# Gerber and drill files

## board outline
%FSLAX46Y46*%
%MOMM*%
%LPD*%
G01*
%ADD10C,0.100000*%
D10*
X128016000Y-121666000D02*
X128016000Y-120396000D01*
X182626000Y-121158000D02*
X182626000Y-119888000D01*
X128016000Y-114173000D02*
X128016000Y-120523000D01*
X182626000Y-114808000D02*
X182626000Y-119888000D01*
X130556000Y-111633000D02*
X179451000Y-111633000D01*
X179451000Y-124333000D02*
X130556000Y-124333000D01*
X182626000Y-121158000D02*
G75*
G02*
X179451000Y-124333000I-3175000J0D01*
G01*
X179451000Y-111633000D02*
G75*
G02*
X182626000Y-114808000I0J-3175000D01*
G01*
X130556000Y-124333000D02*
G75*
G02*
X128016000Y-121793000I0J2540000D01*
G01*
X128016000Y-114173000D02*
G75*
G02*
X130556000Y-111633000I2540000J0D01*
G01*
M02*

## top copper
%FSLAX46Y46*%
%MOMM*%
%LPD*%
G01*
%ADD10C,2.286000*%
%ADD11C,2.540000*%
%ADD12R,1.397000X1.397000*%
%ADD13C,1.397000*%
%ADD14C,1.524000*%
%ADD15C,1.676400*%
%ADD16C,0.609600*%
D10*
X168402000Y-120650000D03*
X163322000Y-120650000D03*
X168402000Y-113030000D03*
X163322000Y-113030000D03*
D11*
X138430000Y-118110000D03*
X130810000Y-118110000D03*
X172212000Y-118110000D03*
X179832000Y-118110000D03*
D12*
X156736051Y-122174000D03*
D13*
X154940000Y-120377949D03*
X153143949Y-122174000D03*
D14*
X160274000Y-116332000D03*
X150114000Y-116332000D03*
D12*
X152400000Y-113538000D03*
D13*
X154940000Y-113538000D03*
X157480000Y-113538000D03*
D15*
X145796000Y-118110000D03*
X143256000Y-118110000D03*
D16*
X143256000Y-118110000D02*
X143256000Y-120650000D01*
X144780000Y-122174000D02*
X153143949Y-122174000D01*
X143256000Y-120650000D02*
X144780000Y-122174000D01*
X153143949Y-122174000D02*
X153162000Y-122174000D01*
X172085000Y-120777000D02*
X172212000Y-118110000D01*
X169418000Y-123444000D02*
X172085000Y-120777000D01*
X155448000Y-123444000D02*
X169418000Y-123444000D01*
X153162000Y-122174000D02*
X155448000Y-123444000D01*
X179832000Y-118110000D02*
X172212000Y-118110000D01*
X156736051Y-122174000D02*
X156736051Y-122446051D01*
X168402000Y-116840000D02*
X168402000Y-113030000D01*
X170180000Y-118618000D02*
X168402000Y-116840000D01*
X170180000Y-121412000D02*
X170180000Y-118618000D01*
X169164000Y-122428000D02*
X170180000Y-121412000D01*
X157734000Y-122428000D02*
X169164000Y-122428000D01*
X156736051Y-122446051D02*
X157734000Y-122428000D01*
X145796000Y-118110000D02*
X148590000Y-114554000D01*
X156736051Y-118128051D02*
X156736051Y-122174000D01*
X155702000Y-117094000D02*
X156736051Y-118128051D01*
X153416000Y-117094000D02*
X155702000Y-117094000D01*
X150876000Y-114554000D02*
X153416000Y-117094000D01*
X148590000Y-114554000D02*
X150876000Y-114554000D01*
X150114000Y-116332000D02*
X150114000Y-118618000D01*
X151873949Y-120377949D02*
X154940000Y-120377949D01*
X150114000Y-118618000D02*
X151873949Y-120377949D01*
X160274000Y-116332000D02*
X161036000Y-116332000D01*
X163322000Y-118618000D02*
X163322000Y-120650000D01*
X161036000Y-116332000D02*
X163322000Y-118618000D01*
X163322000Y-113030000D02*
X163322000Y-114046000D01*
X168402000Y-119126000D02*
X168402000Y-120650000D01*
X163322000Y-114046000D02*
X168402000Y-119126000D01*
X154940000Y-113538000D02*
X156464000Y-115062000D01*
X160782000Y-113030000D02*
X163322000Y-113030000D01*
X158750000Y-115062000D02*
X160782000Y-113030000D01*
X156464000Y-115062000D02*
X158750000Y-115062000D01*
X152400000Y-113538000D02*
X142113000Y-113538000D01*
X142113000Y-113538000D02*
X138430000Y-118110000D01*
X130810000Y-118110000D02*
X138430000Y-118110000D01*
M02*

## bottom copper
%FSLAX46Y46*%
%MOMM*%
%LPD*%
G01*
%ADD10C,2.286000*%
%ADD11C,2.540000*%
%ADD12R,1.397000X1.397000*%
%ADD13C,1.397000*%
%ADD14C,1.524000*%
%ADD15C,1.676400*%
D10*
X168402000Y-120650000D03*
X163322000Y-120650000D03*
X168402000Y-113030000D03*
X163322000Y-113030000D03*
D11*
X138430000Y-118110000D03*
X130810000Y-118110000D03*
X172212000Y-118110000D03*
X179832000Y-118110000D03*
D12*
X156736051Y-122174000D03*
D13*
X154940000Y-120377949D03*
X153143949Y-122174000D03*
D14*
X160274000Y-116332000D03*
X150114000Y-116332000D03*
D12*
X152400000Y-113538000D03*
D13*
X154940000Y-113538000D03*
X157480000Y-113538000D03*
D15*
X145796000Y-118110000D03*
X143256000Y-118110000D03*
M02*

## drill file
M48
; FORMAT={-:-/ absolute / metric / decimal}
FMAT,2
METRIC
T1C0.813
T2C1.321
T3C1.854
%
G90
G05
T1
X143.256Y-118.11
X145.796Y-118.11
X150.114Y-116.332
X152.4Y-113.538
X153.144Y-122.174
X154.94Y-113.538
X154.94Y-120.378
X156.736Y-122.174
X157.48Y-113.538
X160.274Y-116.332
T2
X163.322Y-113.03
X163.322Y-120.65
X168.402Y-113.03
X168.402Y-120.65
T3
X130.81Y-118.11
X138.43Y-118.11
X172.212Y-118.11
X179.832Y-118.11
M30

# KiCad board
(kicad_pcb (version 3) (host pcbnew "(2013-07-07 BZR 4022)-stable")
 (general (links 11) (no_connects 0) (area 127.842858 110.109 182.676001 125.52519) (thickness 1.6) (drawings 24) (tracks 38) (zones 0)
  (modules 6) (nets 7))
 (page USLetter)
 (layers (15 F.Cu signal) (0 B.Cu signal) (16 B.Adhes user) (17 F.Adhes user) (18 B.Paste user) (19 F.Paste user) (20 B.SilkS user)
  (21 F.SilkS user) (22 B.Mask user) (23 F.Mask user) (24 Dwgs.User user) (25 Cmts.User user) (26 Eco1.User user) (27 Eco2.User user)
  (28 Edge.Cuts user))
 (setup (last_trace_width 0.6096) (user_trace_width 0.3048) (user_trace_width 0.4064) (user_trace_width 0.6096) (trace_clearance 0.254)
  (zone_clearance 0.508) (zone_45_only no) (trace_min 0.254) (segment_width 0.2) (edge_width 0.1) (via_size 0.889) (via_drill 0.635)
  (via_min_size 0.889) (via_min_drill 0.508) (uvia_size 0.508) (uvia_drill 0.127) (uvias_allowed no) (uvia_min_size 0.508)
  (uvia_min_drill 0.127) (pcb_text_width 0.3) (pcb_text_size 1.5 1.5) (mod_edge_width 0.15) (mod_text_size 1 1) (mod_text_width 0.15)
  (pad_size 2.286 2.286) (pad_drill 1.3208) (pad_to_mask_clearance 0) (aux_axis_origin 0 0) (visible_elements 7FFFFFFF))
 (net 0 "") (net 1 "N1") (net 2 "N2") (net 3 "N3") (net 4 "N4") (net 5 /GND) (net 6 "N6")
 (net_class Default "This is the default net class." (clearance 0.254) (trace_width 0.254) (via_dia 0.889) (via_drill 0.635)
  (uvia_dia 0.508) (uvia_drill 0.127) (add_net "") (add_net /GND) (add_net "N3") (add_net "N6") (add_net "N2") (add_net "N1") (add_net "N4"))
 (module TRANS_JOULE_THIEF (layer F.Cu) (at 165.862 118.11 180)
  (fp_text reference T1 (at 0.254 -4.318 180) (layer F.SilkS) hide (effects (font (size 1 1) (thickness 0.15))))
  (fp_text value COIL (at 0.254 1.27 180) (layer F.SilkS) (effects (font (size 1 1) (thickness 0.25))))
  (pad 1 thru_hole circle (at -2.54 -2.54 180) (size 2.286 2.286) (drill 1.3208) (layers *.Cu *.Mask F.SilkS) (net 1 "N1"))
  (pad 2 thru_hole circle (at 2.54 -2.54 180) (size 2.286 2.286) (drill 1.3208) (layers *.Cu *.Mask F.SilkS) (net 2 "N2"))
  (pad 3 thru_hole circle (at -2.54 5.08 180) (size 2.286 2.286) (drill 1.3208) (layers *.Cu *.Mask F.SilkS) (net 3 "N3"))
  (pad 4 thru_hole circle (at 2.54 5.08 180) (size 2.286 2.286) (drill 1.3208) (layers *.Cu *.Mask F.SilkS) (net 1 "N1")))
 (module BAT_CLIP (layer F.Cu) (at 155.448 118.11)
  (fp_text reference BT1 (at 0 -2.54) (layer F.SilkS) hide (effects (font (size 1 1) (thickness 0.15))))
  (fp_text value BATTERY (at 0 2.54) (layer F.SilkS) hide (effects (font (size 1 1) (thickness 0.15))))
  (pad 1 thru_hole circle (at -17.018 0) (size 2.54 2.54) (drill 1.8542) (layers *.Cu *.Mask F.SilkS) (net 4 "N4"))
  (pad 1 thru_hole circle (at -24.638 0) (size 2.54 2.54) (drill 1.8542) (layers *.Cu *.Mask F.SilkS) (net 4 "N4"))
  (pad 2 thru_hole circle (at 16.764 0) (size 2.54 2.54) (drill 1.8542) (layers *.Cu *.Mask F.SilkS) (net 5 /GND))
  (pad 2 thru_hole circle (at 24.384 0) (size 2.54 2.54) (drill 1.8542) (layers *.Cu *.Mask F.SilkS) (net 5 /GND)))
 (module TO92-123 (layer F.Cu) (at 154.94 122.174 315)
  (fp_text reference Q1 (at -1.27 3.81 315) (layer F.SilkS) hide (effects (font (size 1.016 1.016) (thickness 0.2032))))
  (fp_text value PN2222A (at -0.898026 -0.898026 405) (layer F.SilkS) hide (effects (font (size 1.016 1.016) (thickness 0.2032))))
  (pad 3 thru_hole rect (at 1.27 -1.27) (size 1.397 1.397) (drill 0.8128) (layers *.Cu *.Mask F.SilkS) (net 3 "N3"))
  (pad 2 thru_hole circle (at -1.27 -1.27 315) (size 1.397 1.397) (drill 0.8128) (layers *.Cu *.Mask F.SilkS) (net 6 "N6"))
  (pad 1 thru_hole circle (at -1.27 1.27 315) (size 1.397 1.397) (drill 0.8128) (layers *.Cu *.Mask F.SilkS) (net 5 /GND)))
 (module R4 (layer F.Cu) (at 155.194 116.332 180) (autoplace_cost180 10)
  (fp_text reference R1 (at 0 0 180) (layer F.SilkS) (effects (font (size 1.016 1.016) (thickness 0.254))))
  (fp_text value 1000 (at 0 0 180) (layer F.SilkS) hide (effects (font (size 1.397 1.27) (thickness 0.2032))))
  (pad 1 thru_hole circle (at -5.08 0 180) (size 1.524 1.524) (drill 0.8128) (layers *.Cu *.Mask F.SilkS) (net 2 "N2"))
  (pad 2 thru_hole circle (at 5.08 0 180) (size 1.524 1.524) (drill 0.8128) (layers *.Cu *.Mask F.SilkS) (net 6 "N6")))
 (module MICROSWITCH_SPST (layer F.Cu) (at 154.94 113.538)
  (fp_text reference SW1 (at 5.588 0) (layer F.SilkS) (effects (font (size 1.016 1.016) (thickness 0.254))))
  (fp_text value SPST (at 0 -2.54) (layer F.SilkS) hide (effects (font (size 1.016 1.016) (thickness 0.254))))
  (pad 1 thru_hole rect (at -2.54 0) (size 1.397 1.397) (drill 0.8128) (layers *.Cu *.Mask F.SilkS) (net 4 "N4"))
  (pad 2 thru_hole circle (at 0 0) (size 1.397 1.397) (drill 0.8128) (layers *.Cu *.Mask F.SilkS) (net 1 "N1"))
  (pad 3 thru_hole circle (at 2.54 0) (size 1.397 1.397) (drill 0.8128) (layers *.Cu *.Mask F.SilkS)))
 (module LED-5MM (layer F.Cu) (at 144.526 118.11 180)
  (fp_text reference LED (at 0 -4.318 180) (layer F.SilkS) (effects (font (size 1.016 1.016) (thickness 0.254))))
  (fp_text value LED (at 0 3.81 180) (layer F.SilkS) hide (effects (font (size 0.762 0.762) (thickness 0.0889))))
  (pad 1 thru_hole circle (at -1.27 0 180) (size 1.6764 1.6764) (drill 0.8128) (layers *.Cu *.Mask F.SilkS) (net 3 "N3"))
  (pad 2 thru_hole circle (at 1.27 0 180) (size 1.6764 1.6764) (drill 0.8128) (layers *.Cu *.Mask F.SilkS) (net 5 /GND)))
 (gr_line (start 128.016 121.666) (end 128.016 120.396) (angle 90) (layer Edge.Cuts) (width 0.1))
 (gr_line (start 182.626 121.158) (end 182.626 119.888) (angle 90) (layer Edge.Cuts) (width 0.1))
 (gr_line (start 128.016 114.173) (end 128.016 120.523) (angle 90) (layer Edge.Cuts) (width 0.1))
 (gr_line (start 182.626 114.808) (end 182.626 119.888) (angle 90) (layer Edge.Cuts) (width 0.1))
 (gr_line (start 130.556 111.633) (end 179.451 111.633) (angle 90) (layer Edge.Cuts) (width 0.1))
 (gr_line (start 179.451 124.333) (end 130.556 124.333) (angle 90) (layer Edge.Cuts) (width 0.1))
 (gr_arc (start 179.451 121.158) (end 182.626 121.158) (angle 90) (layer Edge.Cuts) (width 0.1))
 (gr_arc (start 179.451 114.808) (end 179.451 111.633) (angle 90) (layer Edge.Cuts) (width 0.1))
 (gr_arc (start 130.556 121.793) (end 130.556 124.333) (angle 90) (layer Edge.Cuts) (width 0.1))
 (gr_arc (start 130.556 114.173) (end 128.016 114.173) (angle 90) (layer Edge.Cuts) (width 0.1))
 (segment (start 143.256 118.11) (end 143.256 120.65) (width 0.6096) (layer F.Cu) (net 5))
 (segment (start 144.78 122.174) (end 153.143949 122.174) (width 0.6096) (layer F.Cu) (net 5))
 (segment (start 143.256 120.65) (end 144.78 122.174) (width 0.6096) (layer F.Cu) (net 5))
 (segment (start 153.143949 122.174) (end 153.162 122.174) (width 0.6096) (layer F.Cu) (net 5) (status 30))
 (segment (start 172.085 120.777) (end 172.212 118.11) (width 0.6096) (layer F.Cu) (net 5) (status 20))
 (segment (start 169.418 123.444) (end 172.085 120.777) (width 0.6096) (layer F.Cu) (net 5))
 (segment (start 155.448 123.444) (end 169.418 123.444) (width 0.6096) (layer F.Cu) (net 5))
 (segment (start 153.162 122.174) (end 155.448 123.444) (width 0.6096) (layer F.Cu) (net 5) (status 10))
 (segment (start 179.832 118.11) (end 172.212 118.11) (width 0.6096) (layer F.Cu) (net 5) (status 30))
 (segment (start 156.736051 122.174) (end 156.736051 122.446051) (width 0.6096) (layer F.Cu) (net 3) (status 30))
 (segment (start 168.402 116.84) (end 168.402 113.03) (width 0.6096) (layer F.Cu) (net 3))
 (segment (start 170.18 118.618) (end 168.402 116.84) (width 0.6096) (layer F.Cu) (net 3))
 (segment (start 170.18 121.412) (end 170.18 118.618) (width 0.6096) (layer F.Cu) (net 3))
 (segment (start 169.164 122.428) (end 170.18 121.412) (width 0.6096) (layer F.Cu) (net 3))
 (segment (start 157.734 122.428) (end 169.164 122.428) (width 0.6096) (layer F.Cu) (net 3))
 (segment (start 156.736051 122.446051) (end 157.734 122.428) (width 0.6096) (layer F.Cu) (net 3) (status 10))
 (segment (start 145.796 118.11) (end 148.59 114.554) (width 0.6096) (layer F.Cu) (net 3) (status 10))
 (segment (start 156.736051 118.128051) (end 156.736051 122.174) (width 0.6096) (layer F.Cu) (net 3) (status 20))
 (segment (start 155.702 117.094) (end 156.736051 118.128051) (width 0.6096) (layer F.Cu) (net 3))
 (segment (start 153.416 117.094) (end 155.702 117.094) (width 0.6096) (layer F.Cu) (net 3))
 (segment (start 150.876 114.554) (end 153.416 117.094) (width 0.6096) (layer F.Cu) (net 3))
 (segment (start 148.59 114.554) (end 150.876 114.554) (width 0.6096) (layer F.Cu) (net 3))
 (segment (start 150.114 116.332) (end 150.114 118.618) (width 0.6096) (layer F.Cu) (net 6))
 (segment (start 151.873949 120.377949) (end 154.94 120.377949) (width 0.6096) (layer F.Cu) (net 6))
 (segment (start 150.114 118.618) (end 151.873949 120.377949) (width 0.6096) (layer F.Cu) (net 6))
 (segment (start 160.274 116.332) (end 161.036 116.332) (width 0.6096) (layer F.Cu) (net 2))
 (segment (start 163.322 118.618) (end 163.322 120.65) (width 0.6096) (layer F.Cu) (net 2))
 (segment (start 161.036 116.332) (end 163.322 118.618) (width 0.6096) (layer F.Cu) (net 2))
 (segment (start 163.322 113.03) (end 163.322 114.046) (width 0.6096) (layer F.Cu) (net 1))
 (segment (start 168.402 119.126) (end 168.402 120.65) (width 0.6096) (layer F.Cu) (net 1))
 (segment (start 163.322 114.046) (end 168.402 119.126) (width 0.6096) (layer F.Cu) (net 1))
 (segment (start 154.94 113.538) (end 156.464 115.062) (width 0.6096) (layer F.Cu) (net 1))
 (segment (start 160.782 113.03) (end 163.322 113.03) (width 0.6096) (layer F.Cu) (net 1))
 (segment (start 158.75 115.062) (end 160.782 113.03) (width 0.6096) (layer F.Cu) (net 1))
 (segment (start 156.464 115.062) (end 158.75 115.062) (width 0.6096) (layer F.Cu) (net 1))
 (segment (start 152.4 113.538) (end 142.113 113.538) (width 0.6096) (layer F.Cu) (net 4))
 (segment (start 142.113 113.538) (end 138.43 118.11) (width 0.6096) (layer F.Cu) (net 4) (status 20))
 (segment (start 130.81 118.11) (end 138.43 118.11) (width 0.6096) (layer F.Cu) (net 4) (status 30)))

